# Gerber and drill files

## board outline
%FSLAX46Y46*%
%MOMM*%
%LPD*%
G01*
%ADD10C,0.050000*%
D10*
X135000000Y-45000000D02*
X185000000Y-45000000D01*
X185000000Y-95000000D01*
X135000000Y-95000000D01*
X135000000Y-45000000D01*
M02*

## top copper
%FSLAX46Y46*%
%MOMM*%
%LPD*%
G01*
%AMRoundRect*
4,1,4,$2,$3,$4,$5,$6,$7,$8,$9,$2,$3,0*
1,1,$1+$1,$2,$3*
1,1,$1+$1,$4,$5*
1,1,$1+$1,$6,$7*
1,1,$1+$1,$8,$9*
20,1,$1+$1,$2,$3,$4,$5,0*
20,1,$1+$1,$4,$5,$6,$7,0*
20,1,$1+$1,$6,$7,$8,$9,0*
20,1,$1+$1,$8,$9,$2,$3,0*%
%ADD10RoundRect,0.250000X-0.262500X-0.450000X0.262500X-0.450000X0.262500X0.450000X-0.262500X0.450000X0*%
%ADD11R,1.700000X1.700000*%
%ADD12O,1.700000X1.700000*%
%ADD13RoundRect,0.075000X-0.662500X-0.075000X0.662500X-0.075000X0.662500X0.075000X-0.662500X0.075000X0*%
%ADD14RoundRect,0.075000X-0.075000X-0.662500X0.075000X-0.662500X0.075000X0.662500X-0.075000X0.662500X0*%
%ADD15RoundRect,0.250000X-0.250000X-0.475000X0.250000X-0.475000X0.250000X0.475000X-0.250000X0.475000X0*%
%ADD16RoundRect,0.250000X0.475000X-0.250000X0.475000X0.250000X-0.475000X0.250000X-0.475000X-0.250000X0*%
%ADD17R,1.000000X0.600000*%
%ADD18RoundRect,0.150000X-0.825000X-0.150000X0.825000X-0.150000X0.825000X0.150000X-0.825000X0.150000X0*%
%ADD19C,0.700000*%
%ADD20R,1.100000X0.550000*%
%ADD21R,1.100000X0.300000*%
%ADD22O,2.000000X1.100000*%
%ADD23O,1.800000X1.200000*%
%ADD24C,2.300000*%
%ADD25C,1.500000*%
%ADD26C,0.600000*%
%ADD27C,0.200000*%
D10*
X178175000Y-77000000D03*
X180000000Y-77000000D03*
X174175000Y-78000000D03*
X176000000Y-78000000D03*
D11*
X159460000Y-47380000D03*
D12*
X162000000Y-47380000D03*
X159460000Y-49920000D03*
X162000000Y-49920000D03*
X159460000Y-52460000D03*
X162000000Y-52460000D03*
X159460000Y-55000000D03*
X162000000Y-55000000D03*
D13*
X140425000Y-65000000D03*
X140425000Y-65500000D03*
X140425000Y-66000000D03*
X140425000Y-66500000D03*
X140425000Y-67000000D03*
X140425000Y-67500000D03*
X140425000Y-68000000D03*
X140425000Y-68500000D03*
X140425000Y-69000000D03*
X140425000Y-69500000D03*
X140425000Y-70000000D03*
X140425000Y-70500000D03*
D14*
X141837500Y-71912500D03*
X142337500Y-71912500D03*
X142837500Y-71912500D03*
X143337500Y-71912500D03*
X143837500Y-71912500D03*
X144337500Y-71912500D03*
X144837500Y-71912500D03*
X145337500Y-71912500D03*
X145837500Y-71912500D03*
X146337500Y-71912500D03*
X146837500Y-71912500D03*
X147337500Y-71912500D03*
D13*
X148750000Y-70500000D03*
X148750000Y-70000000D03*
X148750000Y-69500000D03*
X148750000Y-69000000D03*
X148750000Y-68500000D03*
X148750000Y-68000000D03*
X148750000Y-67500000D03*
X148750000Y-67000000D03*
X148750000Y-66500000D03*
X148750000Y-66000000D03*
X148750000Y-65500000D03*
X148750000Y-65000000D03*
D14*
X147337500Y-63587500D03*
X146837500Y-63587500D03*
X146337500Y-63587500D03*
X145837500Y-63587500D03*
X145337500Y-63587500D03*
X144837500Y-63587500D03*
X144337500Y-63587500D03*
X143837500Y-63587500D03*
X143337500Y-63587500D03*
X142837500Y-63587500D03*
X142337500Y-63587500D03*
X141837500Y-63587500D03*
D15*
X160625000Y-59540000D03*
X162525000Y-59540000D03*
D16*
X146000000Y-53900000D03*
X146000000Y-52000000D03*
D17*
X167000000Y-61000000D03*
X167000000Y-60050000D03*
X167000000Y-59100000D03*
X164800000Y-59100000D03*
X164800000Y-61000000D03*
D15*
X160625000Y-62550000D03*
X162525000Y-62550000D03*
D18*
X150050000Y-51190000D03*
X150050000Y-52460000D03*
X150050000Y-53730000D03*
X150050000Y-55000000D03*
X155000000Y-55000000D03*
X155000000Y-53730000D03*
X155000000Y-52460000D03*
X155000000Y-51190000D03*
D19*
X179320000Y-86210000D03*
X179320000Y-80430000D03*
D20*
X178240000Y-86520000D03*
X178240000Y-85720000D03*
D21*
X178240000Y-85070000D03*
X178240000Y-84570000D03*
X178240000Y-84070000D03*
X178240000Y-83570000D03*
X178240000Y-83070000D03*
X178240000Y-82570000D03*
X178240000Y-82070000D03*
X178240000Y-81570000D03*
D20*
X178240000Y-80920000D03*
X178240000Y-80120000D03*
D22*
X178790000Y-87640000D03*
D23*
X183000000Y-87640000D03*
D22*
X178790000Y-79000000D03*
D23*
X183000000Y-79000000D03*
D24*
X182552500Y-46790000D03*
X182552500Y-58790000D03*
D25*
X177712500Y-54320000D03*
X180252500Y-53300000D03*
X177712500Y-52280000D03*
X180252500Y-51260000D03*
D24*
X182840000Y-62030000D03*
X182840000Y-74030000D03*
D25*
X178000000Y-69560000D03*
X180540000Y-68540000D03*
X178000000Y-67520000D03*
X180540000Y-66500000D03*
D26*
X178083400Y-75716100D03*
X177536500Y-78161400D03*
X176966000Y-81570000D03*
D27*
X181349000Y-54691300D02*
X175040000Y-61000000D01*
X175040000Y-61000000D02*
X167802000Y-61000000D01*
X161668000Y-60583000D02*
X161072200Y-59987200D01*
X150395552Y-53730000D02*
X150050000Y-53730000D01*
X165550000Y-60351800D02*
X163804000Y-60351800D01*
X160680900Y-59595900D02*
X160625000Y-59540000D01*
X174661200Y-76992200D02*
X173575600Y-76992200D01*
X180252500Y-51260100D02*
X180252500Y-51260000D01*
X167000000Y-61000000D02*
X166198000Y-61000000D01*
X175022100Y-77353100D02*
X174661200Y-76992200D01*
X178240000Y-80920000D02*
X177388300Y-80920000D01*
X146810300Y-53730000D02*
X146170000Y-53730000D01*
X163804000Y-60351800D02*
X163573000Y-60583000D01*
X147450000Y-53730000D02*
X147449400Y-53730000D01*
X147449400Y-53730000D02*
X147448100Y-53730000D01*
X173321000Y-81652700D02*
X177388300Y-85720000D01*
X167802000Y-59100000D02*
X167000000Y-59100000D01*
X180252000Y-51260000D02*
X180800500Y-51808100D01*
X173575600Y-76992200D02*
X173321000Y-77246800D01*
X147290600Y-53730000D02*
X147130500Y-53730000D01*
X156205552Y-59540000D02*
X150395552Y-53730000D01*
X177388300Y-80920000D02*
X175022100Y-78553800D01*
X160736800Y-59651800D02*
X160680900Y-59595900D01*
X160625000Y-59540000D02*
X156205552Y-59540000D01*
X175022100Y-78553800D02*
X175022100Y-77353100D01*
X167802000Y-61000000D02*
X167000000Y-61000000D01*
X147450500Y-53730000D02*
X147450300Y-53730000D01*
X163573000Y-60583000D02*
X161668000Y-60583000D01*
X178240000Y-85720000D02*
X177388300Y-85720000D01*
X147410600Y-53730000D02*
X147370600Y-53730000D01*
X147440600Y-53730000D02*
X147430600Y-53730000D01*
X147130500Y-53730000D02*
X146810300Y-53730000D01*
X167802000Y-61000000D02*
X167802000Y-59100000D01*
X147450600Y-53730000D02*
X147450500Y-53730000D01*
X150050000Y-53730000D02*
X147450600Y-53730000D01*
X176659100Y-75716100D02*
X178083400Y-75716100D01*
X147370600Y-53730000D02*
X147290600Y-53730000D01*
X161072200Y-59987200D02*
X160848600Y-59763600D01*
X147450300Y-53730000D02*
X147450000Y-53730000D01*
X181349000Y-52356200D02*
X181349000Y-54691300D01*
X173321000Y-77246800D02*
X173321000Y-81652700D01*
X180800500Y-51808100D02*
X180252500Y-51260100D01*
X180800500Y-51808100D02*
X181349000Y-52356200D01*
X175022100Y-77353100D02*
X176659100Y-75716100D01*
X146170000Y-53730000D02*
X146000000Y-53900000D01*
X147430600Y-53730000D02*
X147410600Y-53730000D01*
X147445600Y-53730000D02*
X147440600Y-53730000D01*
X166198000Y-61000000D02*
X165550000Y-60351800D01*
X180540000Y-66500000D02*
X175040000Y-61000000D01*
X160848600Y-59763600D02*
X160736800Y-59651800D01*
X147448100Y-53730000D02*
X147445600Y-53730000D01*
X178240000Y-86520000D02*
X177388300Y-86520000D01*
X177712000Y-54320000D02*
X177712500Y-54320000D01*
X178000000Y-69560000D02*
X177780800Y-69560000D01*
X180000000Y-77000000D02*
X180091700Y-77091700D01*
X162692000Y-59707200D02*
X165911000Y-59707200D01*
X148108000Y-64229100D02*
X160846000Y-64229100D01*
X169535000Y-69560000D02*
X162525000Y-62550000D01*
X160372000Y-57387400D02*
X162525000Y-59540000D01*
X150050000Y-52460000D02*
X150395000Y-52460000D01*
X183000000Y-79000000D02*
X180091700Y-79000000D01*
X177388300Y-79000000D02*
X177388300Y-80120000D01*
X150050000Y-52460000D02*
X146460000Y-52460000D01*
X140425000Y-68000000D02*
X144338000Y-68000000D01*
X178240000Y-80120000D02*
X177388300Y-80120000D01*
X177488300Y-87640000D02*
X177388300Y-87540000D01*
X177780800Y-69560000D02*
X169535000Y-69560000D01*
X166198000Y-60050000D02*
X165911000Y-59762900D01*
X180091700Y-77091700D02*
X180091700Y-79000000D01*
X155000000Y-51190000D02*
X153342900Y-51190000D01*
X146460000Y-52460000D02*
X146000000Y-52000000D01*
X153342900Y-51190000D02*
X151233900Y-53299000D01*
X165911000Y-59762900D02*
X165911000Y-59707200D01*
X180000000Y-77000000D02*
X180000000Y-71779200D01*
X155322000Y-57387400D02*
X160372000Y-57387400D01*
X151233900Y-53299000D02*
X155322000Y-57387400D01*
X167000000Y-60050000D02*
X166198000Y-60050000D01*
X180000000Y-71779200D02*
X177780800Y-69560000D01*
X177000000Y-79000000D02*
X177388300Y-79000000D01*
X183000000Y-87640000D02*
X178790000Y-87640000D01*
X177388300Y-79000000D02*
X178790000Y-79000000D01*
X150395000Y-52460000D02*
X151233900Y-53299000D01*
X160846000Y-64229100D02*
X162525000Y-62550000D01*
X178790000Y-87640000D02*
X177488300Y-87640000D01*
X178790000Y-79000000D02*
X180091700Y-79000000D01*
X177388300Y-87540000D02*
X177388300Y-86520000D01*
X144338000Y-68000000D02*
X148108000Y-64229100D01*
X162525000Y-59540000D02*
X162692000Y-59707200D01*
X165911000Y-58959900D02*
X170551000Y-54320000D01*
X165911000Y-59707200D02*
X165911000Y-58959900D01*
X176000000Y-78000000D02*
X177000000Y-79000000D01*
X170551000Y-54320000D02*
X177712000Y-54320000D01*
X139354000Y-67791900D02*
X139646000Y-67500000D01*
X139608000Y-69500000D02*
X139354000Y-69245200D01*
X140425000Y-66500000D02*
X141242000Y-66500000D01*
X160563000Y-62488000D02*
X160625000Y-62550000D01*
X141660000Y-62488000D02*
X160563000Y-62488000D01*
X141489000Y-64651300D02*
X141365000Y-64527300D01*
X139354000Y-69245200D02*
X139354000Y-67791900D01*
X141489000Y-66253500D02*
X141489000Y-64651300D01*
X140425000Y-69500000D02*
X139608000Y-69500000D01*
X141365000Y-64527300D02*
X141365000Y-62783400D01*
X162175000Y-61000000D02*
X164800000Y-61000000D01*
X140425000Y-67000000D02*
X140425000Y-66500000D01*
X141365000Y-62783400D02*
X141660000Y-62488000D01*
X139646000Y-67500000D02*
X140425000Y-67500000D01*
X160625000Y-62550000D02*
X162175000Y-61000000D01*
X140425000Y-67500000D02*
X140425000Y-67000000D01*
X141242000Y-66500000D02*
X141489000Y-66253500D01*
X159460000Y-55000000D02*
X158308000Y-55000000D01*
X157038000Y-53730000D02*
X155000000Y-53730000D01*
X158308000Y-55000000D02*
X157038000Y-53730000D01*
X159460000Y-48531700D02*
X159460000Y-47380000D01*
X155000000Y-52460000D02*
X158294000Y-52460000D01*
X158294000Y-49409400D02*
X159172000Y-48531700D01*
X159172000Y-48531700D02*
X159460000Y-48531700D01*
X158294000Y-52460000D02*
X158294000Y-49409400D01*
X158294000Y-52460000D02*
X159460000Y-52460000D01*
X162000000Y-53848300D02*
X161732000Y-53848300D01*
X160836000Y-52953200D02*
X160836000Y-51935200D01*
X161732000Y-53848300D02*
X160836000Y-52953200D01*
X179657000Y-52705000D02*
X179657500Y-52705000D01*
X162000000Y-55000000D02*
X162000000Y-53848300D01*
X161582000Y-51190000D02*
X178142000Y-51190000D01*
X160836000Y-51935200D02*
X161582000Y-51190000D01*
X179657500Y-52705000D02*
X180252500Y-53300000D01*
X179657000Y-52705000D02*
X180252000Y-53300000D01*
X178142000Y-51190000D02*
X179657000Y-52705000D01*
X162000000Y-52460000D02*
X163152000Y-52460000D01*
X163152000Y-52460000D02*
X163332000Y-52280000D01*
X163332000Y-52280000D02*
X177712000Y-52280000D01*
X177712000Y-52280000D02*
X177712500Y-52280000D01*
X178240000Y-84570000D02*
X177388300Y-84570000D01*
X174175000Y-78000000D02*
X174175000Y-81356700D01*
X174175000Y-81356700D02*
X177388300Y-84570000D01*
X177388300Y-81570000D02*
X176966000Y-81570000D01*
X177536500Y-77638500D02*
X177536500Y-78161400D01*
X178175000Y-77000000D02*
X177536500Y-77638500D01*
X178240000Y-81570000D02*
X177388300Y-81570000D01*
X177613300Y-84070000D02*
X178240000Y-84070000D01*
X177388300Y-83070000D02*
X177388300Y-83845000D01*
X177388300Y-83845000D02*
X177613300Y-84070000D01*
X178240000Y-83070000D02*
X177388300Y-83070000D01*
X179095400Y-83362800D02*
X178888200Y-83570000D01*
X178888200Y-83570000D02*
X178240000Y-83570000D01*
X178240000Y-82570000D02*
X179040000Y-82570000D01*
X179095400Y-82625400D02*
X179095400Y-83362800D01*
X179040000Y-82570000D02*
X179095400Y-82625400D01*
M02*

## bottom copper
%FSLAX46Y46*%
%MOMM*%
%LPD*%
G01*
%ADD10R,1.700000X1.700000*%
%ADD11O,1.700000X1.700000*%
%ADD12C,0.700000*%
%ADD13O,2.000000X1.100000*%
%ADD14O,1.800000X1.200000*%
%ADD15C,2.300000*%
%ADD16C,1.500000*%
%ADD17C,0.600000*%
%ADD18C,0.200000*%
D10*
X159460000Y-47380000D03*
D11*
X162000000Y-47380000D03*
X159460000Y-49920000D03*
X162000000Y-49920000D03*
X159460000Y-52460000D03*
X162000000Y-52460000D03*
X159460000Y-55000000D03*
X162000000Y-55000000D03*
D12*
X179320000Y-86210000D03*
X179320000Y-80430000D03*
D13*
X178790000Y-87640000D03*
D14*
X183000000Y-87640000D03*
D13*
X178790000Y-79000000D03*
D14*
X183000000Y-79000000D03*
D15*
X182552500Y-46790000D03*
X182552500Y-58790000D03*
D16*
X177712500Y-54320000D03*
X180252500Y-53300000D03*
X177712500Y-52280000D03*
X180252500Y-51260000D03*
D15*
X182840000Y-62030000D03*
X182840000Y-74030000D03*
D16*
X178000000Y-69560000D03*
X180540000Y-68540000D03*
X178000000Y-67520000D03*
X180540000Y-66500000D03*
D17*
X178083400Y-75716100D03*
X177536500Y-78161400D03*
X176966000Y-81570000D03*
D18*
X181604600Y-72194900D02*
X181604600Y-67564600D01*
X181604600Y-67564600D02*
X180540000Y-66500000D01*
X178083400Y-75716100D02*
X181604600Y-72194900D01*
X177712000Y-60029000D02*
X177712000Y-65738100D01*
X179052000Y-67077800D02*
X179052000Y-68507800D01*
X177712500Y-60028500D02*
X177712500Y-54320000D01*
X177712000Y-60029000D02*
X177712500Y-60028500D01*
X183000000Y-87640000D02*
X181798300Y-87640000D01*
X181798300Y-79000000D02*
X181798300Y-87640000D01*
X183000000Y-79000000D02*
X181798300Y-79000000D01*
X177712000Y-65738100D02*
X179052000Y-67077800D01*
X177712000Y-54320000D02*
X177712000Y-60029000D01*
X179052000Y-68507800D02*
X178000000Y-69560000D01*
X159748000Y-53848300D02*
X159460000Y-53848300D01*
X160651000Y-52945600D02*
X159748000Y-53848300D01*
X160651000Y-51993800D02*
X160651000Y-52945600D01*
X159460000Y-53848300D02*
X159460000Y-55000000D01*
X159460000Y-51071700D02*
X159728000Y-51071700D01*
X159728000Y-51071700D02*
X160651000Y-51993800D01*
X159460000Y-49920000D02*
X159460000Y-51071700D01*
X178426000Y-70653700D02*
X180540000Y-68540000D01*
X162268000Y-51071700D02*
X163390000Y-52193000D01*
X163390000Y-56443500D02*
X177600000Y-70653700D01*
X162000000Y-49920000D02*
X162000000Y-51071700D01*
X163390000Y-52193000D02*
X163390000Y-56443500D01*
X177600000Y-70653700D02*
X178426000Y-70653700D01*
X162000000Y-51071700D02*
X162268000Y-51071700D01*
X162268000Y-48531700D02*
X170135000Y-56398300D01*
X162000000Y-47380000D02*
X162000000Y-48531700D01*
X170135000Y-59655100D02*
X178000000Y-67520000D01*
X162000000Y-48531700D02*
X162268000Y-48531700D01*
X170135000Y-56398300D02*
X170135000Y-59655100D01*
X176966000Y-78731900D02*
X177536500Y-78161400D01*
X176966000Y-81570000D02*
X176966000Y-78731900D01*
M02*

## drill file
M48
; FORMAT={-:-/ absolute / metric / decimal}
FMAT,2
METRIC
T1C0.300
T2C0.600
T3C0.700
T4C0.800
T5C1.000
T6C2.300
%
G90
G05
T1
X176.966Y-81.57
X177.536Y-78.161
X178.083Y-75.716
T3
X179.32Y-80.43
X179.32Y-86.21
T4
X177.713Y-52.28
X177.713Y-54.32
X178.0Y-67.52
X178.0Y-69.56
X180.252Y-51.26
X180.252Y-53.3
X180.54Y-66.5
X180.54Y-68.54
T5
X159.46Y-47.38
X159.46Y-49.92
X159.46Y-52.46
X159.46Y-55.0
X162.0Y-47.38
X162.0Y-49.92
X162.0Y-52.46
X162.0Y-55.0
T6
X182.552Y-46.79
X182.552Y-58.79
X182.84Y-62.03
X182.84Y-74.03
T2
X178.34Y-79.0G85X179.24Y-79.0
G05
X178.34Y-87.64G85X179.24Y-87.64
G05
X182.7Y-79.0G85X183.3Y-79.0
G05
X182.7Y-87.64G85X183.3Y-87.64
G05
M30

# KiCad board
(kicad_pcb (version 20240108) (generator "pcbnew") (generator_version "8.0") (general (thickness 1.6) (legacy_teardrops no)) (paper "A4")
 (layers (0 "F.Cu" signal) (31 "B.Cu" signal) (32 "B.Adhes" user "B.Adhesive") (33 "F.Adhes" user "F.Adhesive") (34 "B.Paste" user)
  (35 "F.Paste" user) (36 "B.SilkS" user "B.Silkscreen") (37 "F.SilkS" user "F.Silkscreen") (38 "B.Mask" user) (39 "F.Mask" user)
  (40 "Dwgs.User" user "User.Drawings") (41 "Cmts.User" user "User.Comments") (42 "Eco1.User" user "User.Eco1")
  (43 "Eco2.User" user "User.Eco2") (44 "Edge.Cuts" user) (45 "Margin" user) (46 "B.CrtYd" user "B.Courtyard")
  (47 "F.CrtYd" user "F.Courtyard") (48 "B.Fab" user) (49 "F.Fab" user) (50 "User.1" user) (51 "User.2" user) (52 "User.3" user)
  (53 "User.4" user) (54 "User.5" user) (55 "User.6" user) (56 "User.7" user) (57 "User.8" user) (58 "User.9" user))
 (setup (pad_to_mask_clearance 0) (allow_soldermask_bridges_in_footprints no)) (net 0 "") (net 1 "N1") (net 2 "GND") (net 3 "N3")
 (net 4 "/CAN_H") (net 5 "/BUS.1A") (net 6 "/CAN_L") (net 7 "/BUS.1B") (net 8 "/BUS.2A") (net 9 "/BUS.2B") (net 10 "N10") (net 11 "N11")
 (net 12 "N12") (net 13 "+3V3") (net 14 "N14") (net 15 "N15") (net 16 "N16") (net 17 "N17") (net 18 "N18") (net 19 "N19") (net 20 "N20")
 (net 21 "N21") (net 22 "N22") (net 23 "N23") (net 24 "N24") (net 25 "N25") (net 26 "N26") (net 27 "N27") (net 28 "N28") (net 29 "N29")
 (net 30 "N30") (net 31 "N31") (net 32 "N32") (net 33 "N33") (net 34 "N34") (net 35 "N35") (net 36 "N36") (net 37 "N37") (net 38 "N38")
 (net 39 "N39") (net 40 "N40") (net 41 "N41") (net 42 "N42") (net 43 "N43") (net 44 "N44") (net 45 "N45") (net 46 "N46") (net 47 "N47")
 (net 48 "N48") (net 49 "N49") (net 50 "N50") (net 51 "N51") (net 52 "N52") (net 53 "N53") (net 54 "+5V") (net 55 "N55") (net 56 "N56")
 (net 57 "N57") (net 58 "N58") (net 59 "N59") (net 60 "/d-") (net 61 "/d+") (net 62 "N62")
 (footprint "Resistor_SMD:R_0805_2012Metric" (layer "F.Cu") (at 179.0875 77)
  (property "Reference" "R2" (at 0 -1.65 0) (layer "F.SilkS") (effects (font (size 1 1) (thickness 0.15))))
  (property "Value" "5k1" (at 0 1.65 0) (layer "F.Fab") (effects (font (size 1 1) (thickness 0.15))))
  (pad "1" smd roundrect (at -0.9125 0) (size 1.025 1.4) (layers "F.Cu" "F.Paste" "F.Mask") (roundrect_rratio 0.243902) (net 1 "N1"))
  (pad "2" smd roundrect (at 0.9125 0) (size 1.025 1.4) (layers "F.Cu" "F.Paste" "F.Mask") (roundrect_rratio 0.243902) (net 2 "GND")))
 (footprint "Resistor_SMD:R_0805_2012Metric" (layer "F.Cu") (at 175.0875 78)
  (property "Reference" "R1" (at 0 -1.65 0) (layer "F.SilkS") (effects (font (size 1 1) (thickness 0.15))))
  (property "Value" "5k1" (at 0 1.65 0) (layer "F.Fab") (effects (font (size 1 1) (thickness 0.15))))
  (pad "1" smd roundrect (at -0.9125 0) (size 1.025 1.4) (layers "F.Cu" "F.Paste" "F.Mask") (roundrect_rratio 0.243902) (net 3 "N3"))
  (pad "2" smd roundrect (at 0.9125 0) (size 1.025 1.4) (layers "F.Cu" "F.Paste" "F.Mask") (roundrect_rratio 0.243902) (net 2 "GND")))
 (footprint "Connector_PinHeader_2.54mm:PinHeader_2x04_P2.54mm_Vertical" (layer "F.Cu") (at 159.46 47.38)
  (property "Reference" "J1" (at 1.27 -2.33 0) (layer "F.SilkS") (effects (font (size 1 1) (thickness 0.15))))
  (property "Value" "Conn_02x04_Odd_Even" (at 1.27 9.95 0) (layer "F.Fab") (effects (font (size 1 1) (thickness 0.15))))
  (pad "1" thru_hole rect (at 0 0) (size 1.7 1.7) (drill 1) (layers "*.Cu" "*.Mask") (remove_unused_layers no) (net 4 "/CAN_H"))
  (pad "2" thru_hole oval (at 2.54 0) (size 1.7 1.7) (drill 1) (layers "*.Cu" "*.Mask") (remove_unused_layers no) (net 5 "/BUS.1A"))
  (pad "3" thru_hole oval (at 0 2.54) (size 1.7 1.7) (drill 1) (layers "*.Cu" "*.Mask") (remove_unused_layers no) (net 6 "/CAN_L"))
  (pad "4" thru_hole oval (at 2.54 2.54) (size 1.7 1.7) (drill 1) (layers "*.Cu" "*.Mask") (remove_unused_layers no) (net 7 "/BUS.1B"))
  (pad "5" thru_hole oval (at 0 5.08) (size 1.7 1.7) (drill 1) (layers "*.Cu" "*.Mask") (remove_unused_layers no) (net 4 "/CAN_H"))
  (pad "6" thru_hole oval (at 2.54 5.08) (size 1.7 1.7) (drill 1) (layers "*.Cu" "*.Mask") (remove_unused_layers no) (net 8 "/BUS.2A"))
  (pad "7" thru_hole oval (at 0 7.62) (size 1.7 1.7) (drill 1) (layers "*.Cu" "*.Mask") (remove_unused_layers no) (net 6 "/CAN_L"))
  (pad "8" thru_hole oval (at 2.54 7.62) (size 1.7 1.7) (drill 1) (layers "*.Cu" "*.Mask") (remove_unused_layers no) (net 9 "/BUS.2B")))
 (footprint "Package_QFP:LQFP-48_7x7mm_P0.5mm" (layer "F.Cu") (at 144.5875 67.75)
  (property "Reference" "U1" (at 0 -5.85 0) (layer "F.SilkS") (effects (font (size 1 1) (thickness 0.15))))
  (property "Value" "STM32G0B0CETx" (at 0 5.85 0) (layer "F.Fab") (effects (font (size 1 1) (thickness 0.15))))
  (pad "1" smd roundrect (at -4.1625 -2.75) (size 1.475 0.3) (layers "F.Cu" "F.Paste" "F.Mask") (roundrect_rratio 0.25) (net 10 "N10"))
  (pad "2" smd roundrect (at -4.1625 -2.25) (size 1.475 0.3) (layers "F.Cu" "F.Paste" "F.Mask") (roundrect_rratio 0.25) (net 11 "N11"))
  (pad "3" smd roundrect (at -4.1625 -1.75) (size 1.475 0.3) (layers "F.Cu" "F.Paste" "F.Mask") (roundrect_rratio 0.25) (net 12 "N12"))
  (pad "4" smd roundrect (at -4.1625 -1.25) (size 1.475 0.3) (layers "F.Cu" "F.Paste" "F.Mask") (roundrect_rratio 0.25) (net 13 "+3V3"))
  (pad "5" smd roundrect (at -4.1625 -0.75) (size 1.475 0.3) (layers "F.Cu" "F.Paste" "F.Mask") (roundrect_rratio 0.25) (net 13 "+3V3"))
  (pad "6" smd roundrect (at -4.1625 -0.25) (size 1.475 0.3) (layers "F.Cu" "F.Paste" "F.Mask") (roundrect_rratio 0.25) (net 13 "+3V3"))
  (pad "7" smd roundrect (at -4.1625 0.25) (size 1.475 0.3) (layers "F.Cu" "F.Paste" "F.Mask") (roundrect_rratio 0.25) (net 2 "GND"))
  (pad "8" smd roundrect (at -4.1625 0.75) (size 1.475 0.3) (layers "F.Cu" "F.Paste" "F.Mask") (roundrect_rratio 0.25) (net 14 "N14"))
  (pad "9" smd roundrect (at -4.1625 1.25) (size 1.475 0.3) (layers "F.Cu" "F.Paste" "F.Mask") (roundrect_rratio 0.25) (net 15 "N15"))
  (pad "10" smd roundrect (at -4.1625 1.75) (size 1.475 0.3) (layers "F.Cu" "F.Paste" "F.Mask") (roundrect_rratio 0.25) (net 13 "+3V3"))
  (pad "11" smd roundrect (at -4.1625 2.25) (size 1.475 0.3) (layers "F.Cu" "F.Paste" "F.Mask") (roundrect_rratio 0.25) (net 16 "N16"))
  (pad "12" smd roundrect (at -4.1625 2.75) (size 1.475 0.3) (layers "F.Cu" "F.Paste" "F.Mask") (roundrect_rratio 0.25) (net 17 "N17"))
  (pad "13" smd roundrect (at -2.75 4.1625) (size 0.3 1.475) (layers "F.Cu" "F.Paste" "F.Mask") (roundrect_rratio 0.25) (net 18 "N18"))
  (pad "14" smd roundrect (at -2.25 4.1625) (size 0.3 1.475) (layers "F.Cu" "F.Paste" "F.Mask") (roundrect_rratio 0.25) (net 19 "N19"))
  (pad "15" smd roundrect (at -1.75 4.1625) (size 0.3 1.475) (layers "F.Cu" "F.Paste" "F.Mask") (roundrect_rratio 0.25) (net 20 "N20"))
  (pad "16" smd roundrect (at -1.25 4.1625) (size 0.3 1.475) (layers "F.Cu" "F.Paste" "F.Mask") (roundrect_rratio 0.25) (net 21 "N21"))
  (pad "17" smd roundrect (at -0.75 4.1625) (size 0.3 1.475) (layers "F.Cu" "F.Paste" "F.Mask") (roundrect_rratio 0.25) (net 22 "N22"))
  (pad "18" smd roundrect (at -0.25 4.1625) (size 0.3 1.475) (layers "F.Cu" "F.Paste" "F.Mask") (roundrect_rratio 0.25) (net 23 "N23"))
  (pad "19" smd roundrect (at 0.25 4.1625) (size 0.3 1.475) (layers "F.Cu" "F.Paste" "F.Mask") (roundrect_rratio 0.25) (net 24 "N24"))
  (pad "20" smd roundrect (at 0.75 4.1625) (size 0.3 1.475) (layers "F.Cu" "F.Paste" "F.Mask") (roundrect_rratio 0.25) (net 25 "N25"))
  (pad "21" smd roundrect (at 1.25 4.1625) (size 0.3 1.475) (layers "F.Cu" "F.Paste" "F.Mask") (roundrect_rratio 0.25) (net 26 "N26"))
  (pad "22" smd roundrect (at 1.75 4.1625) (size 0.3 1.475) (layers "F.Cu" "F.Paste" "F.Mask") (roundrect_rratio 0.25) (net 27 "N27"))
  (pad "23" smd roundrect (at 2.25 4.1625) (size 0.3 1.475) (layers "F.Cu" "F.Paste" "F.Mask") (roundrect_rratio 0.25) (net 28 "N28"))
  (pad "24" smd roundrect (at 2.75 4.1625) (size 0.3 1.475) (layers "F.Cu" "F.Paste" "F.Mask") (roundrect_rratio 0.25) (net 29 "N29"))
  (pad "25" smd roundrect (at 4.1625 2.75) (size 1.475 0.3) (layers "F.Cu" "F.Paste" "F.Mask") (roundrect_rratio 0.25) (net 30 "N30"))
  (pad "26" smd roundrect (at 4.1625 2.25) (size 1.475 0.3) (layers "F.Cu" "F.Paste" "F.Mask") (roundrect_rratio 0.25) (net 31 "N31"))
  (pad "27" smd roundrect (at 4.1625 1.75) (size 1.475 0.3) (layers "F.Cu" "F.Paste" "F.Mask") (roundrect_rratio 0.25) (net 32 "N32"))
  (pad "28" smd roundrect (at 4.1625 1.25) (size 1.475 0.3) (layers "F.Cu" "F.Paste" "F.Mask") (roundrect_rratio 0.25) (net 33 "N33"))
  (pad "29" smd roundrect (at 4.1625 0.75) (size 1.475 0.3) (layers "F.Cu" "F.Paste" "F.Mask") (roundrect_rratio 0.25) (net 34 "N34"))
  (pad "30" smd roundrect (at 4.1625 0.25) (size 1.475 0.3) (layers "F.Cu" "F.Paste" "F.Mask") (roundrect_rratio 0.25) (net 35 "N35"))
  (pad "31" smd roundrect (at 4.1625 -0.25) (size 1.475 0.3) (layers "F.Cu" "F.Paste" "F.Mask") (roundrect_rratio 0.25) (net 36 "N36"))
  (pad "32" smd roundrect (at 4.1625 -0.75) (size 1.475 0.3) (layers "F.Cu" "F.Paste" "F.Mask") (roundrect_rratio 0.25) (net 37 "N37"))
  (pad "33" smd roundrect (at 4.1625 -1.25) (size 1.475 0.3) (layers "F.Cu" "F.Paste" "F.Mask") (roundrect_rratio 0.25) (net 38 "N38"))
  (pad "34" smd roundrect (at 4.1625 -1.75) (size 1.475 0.3) (layers "F.Cu" "F.Paste" "F.Mask") (roundrect_rratio 0.25) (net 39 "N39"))
  (pad "35" smd roundrect (at 4.1625 -2.25) (size 1.475 0.3) (layers "F.Cu" "F.Paste" "F.Mask") (roundrect_rratio 0.25) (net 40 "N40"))
  (pad "36" smd roundrect (at 4.1625 -2.75) (size 1.475 0.3) (layers "F.Cu" "F.Paste" "F.Mask") (roundrect_rratio 0.25) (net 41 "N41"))
  (pad "37" smd roundrect (at 2.75 -4.1625) (size 0.3 1.475) (layers "F.Cu" "F.Paste" "F.Mask") (roundrect_rratio 0.25) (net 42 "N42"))
  (pad "38" smd roundrect (at 2.25 -4.1625) (size 0.3 1.475) (layers "F.Cu" "F.Paste" "F.Mask") (roundrect_rratio 0.25) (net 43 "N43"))
  (pad "39" smd roundrect (at 1.75 -4.1625) (size 0.3 1.475) (layers "F.Cu" "F.Paste" "F.Mask") (roundrect_rratio 0.25) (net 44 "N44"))
  (pad "40" smd roundrect (at 1.25 -4.1625) (size 0.3 1.475) (layers "F.Cu" "F.Paste" "F.Mask") (roundrect_rratio 0.25) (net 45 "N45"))
  (pad "41" smd roundrect (at 0.75 -4.1625) (size 0.3 1.475) (layers "F.Cu" "F.Paste" "F.Mask") (roundrect_rratio 0.25) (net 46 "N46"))
  (pad "42" smd roundrect (at 0.25 -4.1625) (size 0.3 1.475) (layers "F.Cu" "F.Paste" "F.Mask") (roundrect_rratio 0.25) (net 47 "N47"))
  (pad "43" smd roundrect (at -0.25 -4.1625) (size 0.3 1.475) (layers "F.Cu" "F.Paste" "F.Mask") (roundrect_rratio 0.25) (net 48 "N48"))
  (pad "44" smd roundrect (at -0.75 -4.1625) (size 0.3 1.475) (layers "F.Cu" "F.Paste" "F.Mask") (roundrect_rratio 0.25) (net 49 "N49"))
  (pad "45" smd roundrect (at -1.25 -4.1625) (size 0.3 1.475) (layers "F.Cu" "F.Paste" "F.Mask") (roundrect_rratio 0.25) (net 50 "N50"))
  (pad "46" smd roundrect (at -1.75 -4.1625) (size 0.3 1.475) (layers "F.Cu" "F.Paste" "F.Mask") (roundrect_rratio 0.25) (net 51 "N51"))
  (pad "47" smd roundrect (at -2.25 -4.1625) (size 0.3 1.475) (layers "F.Cu" "F.Paste" "F.Mask") (roundrect_rratio 0.25) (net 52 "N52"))
  (pad "48" smd roundrect (at -2.75 -4.1625) (size 0.3 1.475) (layers "F.Cu" "F.Paste" "F.Mask") (roundrect_rratio 0.25) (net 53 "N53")))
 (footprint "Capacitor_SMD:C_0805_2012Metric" (layer "F.Cu") (at 161.575 59.54)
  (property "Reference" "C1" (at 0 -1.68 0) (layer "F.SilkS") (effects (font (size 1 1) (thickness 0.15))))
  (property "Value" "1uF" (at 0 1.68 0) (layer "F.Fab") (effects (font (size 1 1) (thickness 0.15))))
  (pad "1" smd roundrect (at -0.95 0) (size 1 1.45) (layers "F.Cu" "F.Paste" "F.Mask") (roundrect_rratio 0.25) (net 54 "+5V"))
  (pad "2" smd roundrect (at 0.95 0) (size 1 1.45) (layers "F.Cu" "F.Paste" "F.Mask") (roundrect_rratio 0.25) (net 2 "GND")))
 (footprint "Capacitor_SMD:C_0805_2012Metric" (layer "F.Cu") (at 146 52.95 90)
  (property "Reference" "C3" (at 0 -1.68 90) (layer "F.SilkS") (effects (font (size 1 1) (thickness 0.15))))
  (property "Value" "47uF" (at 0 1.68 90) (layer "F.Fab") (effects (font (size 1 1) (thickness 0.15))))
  (pad "1" smd roundrect (at -0.95 0 90) (size 1 1.45) (layers "F.Cu" "F.Paste" "F.Mask") (roundrect_rratio 0.25) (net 54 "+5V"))
  (pad "2" smd roundrect (at 0.95 0 90) (size 1 1.45) (layers "F.Cu" "F.Paste" "F.Mask") (roundrect_rratio 0.25) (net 2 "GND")))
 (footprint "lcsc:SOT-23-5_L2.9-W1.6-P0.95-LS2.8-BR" (layer "F.Cu") (at 165.9 60.05)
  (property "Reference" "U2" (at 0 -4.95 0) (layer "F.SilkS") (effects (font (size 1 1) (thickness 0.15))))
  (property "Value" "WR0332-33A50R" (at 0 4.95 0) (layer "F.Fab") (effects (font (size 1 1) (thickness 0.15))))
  (pad "1" smd rect (at 1.1 0.95 90) (size 0.6 1) (layers "F.Cu" "F.Paste" "F.Mask") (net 54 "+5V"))
  (pad "2" smd rect (at 1.1 0 90) (size 0.6 1) (layers "F.Cu" "F.Paste" "F.Mask") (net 2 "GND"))
  (pad "3" smd rect (at 1.1 -0.95 90) (size 0.6 1) (layers "F.Cu" "F.Paste" "F.Mask") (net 54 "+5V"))
  (pad "4" smd rect (at -1.1 -0.95 90) (size 0.6 1) (layers "F.Cu" "F.Paste" "F.Mask") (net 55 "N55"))
  (pad "5" smd rect (at -1.1 0.95 90) (size 0.6 1) (layers "F.Cu" "F.Paste" "F.Mask") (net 13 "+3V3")))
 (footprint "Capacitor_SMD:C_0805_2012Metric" (layer "F.Cu") (at 161.575 62.55)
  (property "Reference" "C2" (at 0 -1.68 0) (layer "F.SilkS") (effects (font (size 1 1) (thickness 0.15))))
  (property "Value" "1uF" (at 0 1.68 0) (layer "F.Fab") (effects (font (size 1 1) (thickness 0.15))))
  (pad "1" smd roundrect (at -0.95 0) (size 1 1.45) (layers "F.Cu" "F.Paste" "F.Mask") (roundrect_rratio 0.25) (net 13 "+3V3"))
  (pad "2" smd roundrect (at 0.95 0) (size 1 1.45) (layers "F.Cu" "F.Paste" "F.Mask") (roundrect_rratio 0.25) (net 2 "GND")))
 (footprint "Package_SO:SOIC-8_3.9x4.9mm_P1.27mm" (layer "F.Cu") (at 152.525 53.095)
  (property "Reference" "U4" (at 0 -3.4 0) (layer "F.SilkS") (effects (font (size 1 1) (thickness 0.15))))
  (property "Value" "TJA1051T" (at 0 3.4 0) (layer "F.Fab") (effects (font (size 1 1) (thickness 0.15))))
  (pad "1" smd roundrect (at -2.475 -1.905) (size 1.95 0.6) (layers "F.Cu" "F.Paste" "F.Mask") (roundrect_rratio 0.25) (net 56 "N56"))
  (pad "2" smd roundrect (at -2.475 -0.635) (size 1.95 0.6) (layers "F.Cu" "F.Paste" "F.Mask") (roundrect_rratio 0.25) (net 2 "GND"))
  (pad "3" smd roundrect (at -2.475 0.635) (size 1.95 0.6) (layers "F.Cu" "F.Paste" "F.Mask") (roundrect_rratio 0.25) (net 54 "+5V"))
  (pad "4" smd roundrect (at -2.475 1.905) (size 1.95 0.6) (layers "F.Cu" "F.Paste" "F.Mask") (roundrect_rratio 0.25) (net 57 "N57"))
  (pad "5" smd roundrect (at 2.475 1.905) (size 1.95 0.6) (layers "F.Cu" "F.Paste" "F.Mask") (roundrect_rratio 0.25) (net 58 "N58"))
  (pad "6" smd roundrect (at 2.475 0.635) (size 1.95 0.6) (layers "F.Cu" "F.Paste" "F.Mask") (roundrect_rratio 0.25) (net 6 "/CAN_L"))
  (pad "7" smd roundrect (at 2.475 -0.635) (size 1.95 0.6) (layers "F.Cu" "F.Paste" "F.Mask") (roundrect_rratio 0.25) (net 4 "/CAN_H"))
  (pad "8" smd roundrect (at 2.475 -1.905) (size 1.95 0.6) (layers "F.Cu" "F.Paste" "F.Mask") (roundrect_rratio 0.25) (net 2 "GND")))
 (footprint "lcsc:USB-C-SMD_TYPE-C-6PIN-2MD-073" (layer "F.Cu") (at 180.62 83.32 90)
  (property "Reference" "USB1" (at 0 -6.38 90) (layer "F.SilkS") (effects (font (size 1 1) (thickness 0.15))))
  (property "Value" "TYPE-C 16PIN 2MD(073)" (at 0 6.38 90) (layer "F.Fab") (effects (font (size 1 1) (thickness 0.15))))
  (pad "" thru_hole circle (at -2.89 -1.3 90) (size 0.7 0.7) (drill 0.7) (layers "*.Cu" "*.Mask") (remove_unused_layers no))
  (pad "" thru_hole circle (at 2.89 -1.3 90) (size 0.7 0.7) (drill 0.7) (layers "*.Cu" "*.Mask") (remove_unused_layers no))
  (pad "1" smd rect (at -3.2 -2.38 90) (size 0.55 1.1) (layers "F.Cu" "F.Paste" "F.Mask") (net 2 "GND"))
  (pad "2" smd rect (at -2.4 -2.38 90) (size 0.55 1.1) (layers "F.Cu" "F.Paste" "F.Mask") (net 54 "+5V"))
  (pad "3" smd rect (at -1.75 -2.38 90) (size 0.3 1.1) (layers "F.Cu" "F.Paste" "F.Mask") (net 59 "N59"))
  (pad "4" smd rect (at -1.25 -2.38 90) (size 0.3 1.1) (layers "F.Cu" "F.Paste" "F.Mask") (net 3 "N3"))
  (pad "5" smd rect (at -0.75 -2.38 90) (size 0.3 1.1) (layers "F.Cu" "F.Paste" "F.Mask") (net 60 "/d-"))
  (pad "6" smd rect (at -0.25 -2.38 90) (size 0.3 1.1) (layers "F.Cu" "F.Paste" "F.Mask") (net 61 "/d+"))
  (pad "7" smd rect (at 0.25 -2.38 90) (size 0.3 1.1) (layers "F.Cu" "F.Paste" "F.Mask") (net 60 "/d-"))
  (pad "8" smd rect (at 0.75 -2.38 90) (size 0.3 1.1) (layers "F.Cu" "F.Paste" "F.Mask") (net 61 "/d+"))
  (pad "9" smd rect (at 1.25 -2.38 90) (size 0.3 1.1) (layers "F.Cu" "F.Paste" "F.Mask") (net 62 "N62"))
  (pad "10" smd rect (at 1.75 -2.38 90) (size 0.3 1.1) (layers "F.Cu" "F.Paste" "F.Mask") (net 1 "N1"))
  (pad "11" smd rect (at 2.4 -2.38 90) (size 0.55 1.1) (layers "F.Cu" "F.Paste" "F.Mask") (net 54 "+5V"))
  (pad "12" smd rect (at 3.2 -2.38 90) (size 0.55 1.1) (layers "F.Cu" "F.Paste" "F.Mask") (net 2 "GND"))
  (pad "13" thru_hole oval (at -4.32 -1.83 90) (size 1.1 2) (drill oval 0.599999 1.499997) (layers "*.Cu" "*.Mask")
   (remove_unused_layers no) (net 2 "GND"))
  (pad "13" thru_hole oval (at -4.32 2.38 90) (size 1.2 1.8) (drill oval 0.599999 1.199998) (layers "*.Cu" "*.Mask")
   (remove_unused_layers no) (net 2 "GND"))
  (pad "14" thru_hole oval (at 4.32 -1.83 90) (size 1.1 2) (drill oval 0.599999 1.500022) (layers "*.Cu" "*.Mask") (remove_unused_layers no)
   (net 2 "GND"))
  (pad "14" thru_hole oval (at 4.32 2.38 90) (size 1.2 1.8) (drill oval 0.599999 1.199998) (layers "*.Cu" "*.Mask")
   (remove_unused_layers no) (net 2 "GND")))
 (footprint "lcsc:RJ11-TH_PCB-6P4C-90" (layer "F.Cu") (at 178.9825 52.79 -90)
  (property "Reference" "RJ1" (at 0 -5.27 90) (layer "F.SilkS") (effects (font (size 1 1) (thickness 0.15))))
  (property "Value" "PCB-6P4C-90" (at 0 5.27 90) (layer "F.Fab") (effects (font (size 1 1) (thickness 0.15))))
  (pad "" thru_hole circle (at -6 -3.57 270) (size 2.3 2.3) (drill 2.3) (layers "*.Cu" "*.Mask") (remove_unused_layers no))
  (pad "" thru_hole circle (at 6 -3.57 270) (size 2.3 2.3) (drill 2.3) (layers "*.Cu" "*.Mask") (remove_unused_layers no))
  (pad "1" thru_hole circle (at 1.53 1.27 270) (size 1.5 1.5) (drill 0.799998) (layers "*.Cu" "*.Mask") (remove_unused_layers no)
   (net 2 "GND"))
  (pad "2" thru_hole circle (at 0.51 -1.27 270) (size 1.5 1.5) (drill 0.799998) (layers "*.Cu" "*.Mask") (remove_unused_layers no)
   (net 9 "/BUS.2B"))
  (pad "3" thru_hole circle (at -0.51 1.27 270) (size 1.5 1.5) (drill 0.799998) (layers "*.Cu" "*.Mask") (remove_unused_layers no)
   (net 8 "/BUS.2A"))
  (pad "4" thru_hole circle (at -1.53 -1.27 270) (size 1.5 1.5) (drill 0.799998) (layers "*.Cu" "*.Mask") (remove_unused_layers no)
   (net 54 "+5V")))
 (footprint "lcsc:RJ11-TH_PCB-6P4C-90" (layer "F.Cu") (at 179.27 68.03 -90)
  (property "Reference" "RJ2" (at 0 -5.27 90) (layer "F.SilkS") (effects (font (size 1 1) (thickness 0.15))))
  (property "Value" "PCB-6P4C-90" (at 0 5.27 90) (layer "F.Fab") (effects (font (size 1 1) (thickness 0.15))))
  (pad "" thru_hole circle (at -6 -3.57 270) (size 2.3 2.3) (drill 2.3) (layers "*.Cu" "*.Mask") (remove_unused_layers no))
  (pad "" thru_hole circle (at 6 -3.57 270) (size 2.3 2.3) (drill 2.3) (layers "*.Cu" "*.Mask") (remove_unused_layers no))
  (pad "1" thru_hole circle (at 1.53 1.27 270) (size 1.5 1.5) (drill 0.799998) (layers "*.Cu" "*.Mask") (remove_unused_layers no)
   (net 2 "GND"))
  (pad "2" thru_hole circle (at 0.51 -1.27 270) (size 1.5 1.5) (drill 0.799998) (layers "*.Cu" "*.Mask") (remove_unused_layers no)
   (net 7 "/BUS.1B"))
  (pad "3" thru_hole circle (at -0.51 1.27 270) (size 1.5 1.5) (drill 0.799998) (layers "*.Cu" "*.Mask") (remove_unused_layers no)
   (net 5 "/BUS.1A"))
  (pad "4" thru_hole circle (at -1.53 -1.27 270) (size 1.5 1.5) (drill 0.799998) (layers "*.Cu" "*.Mask") (remove_unused_layers no)
   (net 54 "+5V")))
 (gr_rect (start 135 45) (end 185 95) (stroke (width 0.05) (type default)) (fill none) (layer "Edge.Cuts"))
 (segment (start 181.349 54.6913) (end 175.04 61) (width 0.2) (layer "F.Cu") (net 54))
 (segment (start 175.04 61) (end 167.802 61) (width 0.2) (layer "F.Cu") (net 54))
 (segment (start 161.668 60.583) (end 161.0722 59.9872) (width 0.2) (layer "F.Cu") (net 54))
 (segment (start 150.395552 53.73) (end 150.05 53.73) (width 0.2) (layer "F.Cu") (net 54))
 (segment (start 165.55 60.3518) (end 163.804 60.3518) (width 0.2) (layer "F.Cu") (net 54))
 (segment (start 160.6809 59.5959) (end 160.625 59.54) (width 0.2) (layer "F.Cu") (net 54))
 (segment (start 174.6612 76.9922) (end 173.5756 76.9922) (width 0.2) (layer "F.Cu") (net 54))
 (segment (start 180.2525 51.2601) (end 180.2525 51.26) (width 0.2) (layer "F.Cu") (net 54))
 (segment (start 167 61) (end 166.198 61) (width 0.2) (layer "F.Cu") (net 54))
 (segment (start 175.0221 77.3531) (end 174.6612 76.9922) (width 0.2) (layer "F.Cu") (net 54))
 (segment (start 178.24 80.92) (end 177.3883 80.92) (width 0.2) (layer "F.Cu") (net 54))
 (segment (start 146.8103 53.73) (end 146.17 53.73) (width 0.2) (layer "F.Cu") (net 54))
 (segment (start 163.804 60.3518) (end 163.573 60.583) (width 0.2) (layer "F.Cu") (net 54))
 (segment (start 147.45 53.73) (end 147.4494 53.73) (width 0.2) (layer "F.Cu") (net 54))
 (segment (start 147.4494 53.73) (end 147.4481 53.73) (width 0.2) (layer "F.Cu") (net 54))
 (segment (start 173.321 81.6527) (end 177.3883 85.72) (width 0.2) (layer "F.Cu") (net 54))
 (segment (start 167.802 59.1) (end 167 59.1) (width 0.2) (layer "F.Cu") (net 54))
 (segment (start 180.252 51.26) (end 180.8005 51.8081) (width 0.2) (layer "F.Cu") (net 54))
 (segment (start 173.5756 76.9922) (end 173.321 77.2468) (width 0.2) (layer "F.Cu") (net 54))
 (segment (start 147.2906 53.73) (end 147.1305 53.73) (width 0.2) (layer "F.Cu") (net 54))
 (segment (start 156.205552 59.54) (end 150.395552 53.73) (width 0.2) (layer "F.Cu") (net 54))
 (segment (start 177.3883 80.92) (end 175.0221 78.5538) (width 0.2) (layer "F.Cu") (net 54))
 (segment (start 160.7368 59.6518) (end 160.6809 59.5959) (width 0.2) (layer "F.Cu") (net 54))
 (segment (start 160.625 59.54) (end 156.205552 59.54) (width 0.2) (layer "F.Cu") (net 54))
 (segment (start 175.0221 78.5538) (end 175.0221 77.3531) (width 0.2) (layer "F.Cu") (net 54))
 (segment (start 167.802 61) (end 167 61) (width 0.2) (layer "F.Cu") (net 54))
 (segment (start 147.4505 53.73) (end 147.4503 53.73) (width 0.2) (layer "F.Cu") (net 54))
 (segment (start 163.573 60.583) (end 161.668 60.583) (width 0.2) (layer "F.Cu") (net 54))
 (segment (start 178.24 85.72) (end 177.3883 85.72) (width 0.2) (layer "F.Cu") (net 54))
 (segment (start 147.4106 53.73) (end 147.3706 53.73) (width 0.2) (layer "F.Cu") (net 54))
 (segment (start 147.4406 53.73) (end 147.4306 53.73) (width 0.2) (layer "F.Cu") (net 54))
 (segment (start 147.1305 53.73) (end 146.8103 53.73) (width 0.2) (layer "F.Cu") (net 54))
 (segment (start 167.802 61) (end 167.802 59.1) (width 0.2) (layer "F.Cu") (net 54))
 (segment (start 147.4506 53.73) (end 147.4505 53.73) (width 0.2) (layer "F.Cu") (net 54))
 (segment (start 150.05 53.73) (end 147.4506 53.73) (width 0.2) (layer "F.Cu") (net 54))
 (segment (start 176.6591 75.7161) (end 178.0834 75.7161) (width 0.2) (layer "F.Cu") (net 54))
 (segment (start 147.3706 53.73) (end 147.2906 53.73) (width 0.2) (layer "F.Cu") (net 54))
 (segment (start 161.0722 59.9872) (end 160.8486 59.7636) (width 0.2) (layer "F.Cu") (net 54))
 (segment (start 147.4503 53.73) (end 147.45 53.73) (width 0.2) (layer "F.Cu") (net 54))
 (segment (start 181.349 52.3562) (end 181.349 54.6913) (width 0.2) (layer "F.Cu") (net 54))
 (segment (start 173.321 77.2468) (end 173.321 81.6527) (width 0.2) (layer "F.Cu") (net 54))
 (segment (start 180.8005 51.8081) (end 180.2525 51.2601) (width 0.2) (layer "F.Cu") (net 54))
 (segment (start 180.8005 51.8081) (end 181.349 52.3562) (width 0.2) (layer "F.Cu") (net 54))
 (segment (start 175.0221 77.3531) (end 176.6591 75.7161) (width 0.2) (layer "F.Cu") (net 54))
 (segment (start 146.17 53.73) (end 146 53.9) (width 0.2) (layer "F.Cu") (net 54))
 (segment (start 147.4306 53.73) (end 147.4106 53.73) (width 0.2) (layer "F.Cu") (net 54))
 (segment (start 147.4456 53.73) (end 147.4406 53.73) (width 0.2) (layer "F.Cu") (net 54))
 (segment (start 166.198 61) (end 165.55 60.3518) (width 0.2) (layer "F.Cu") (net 54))
 (segment (start 180.54 66.5) (end 175.04 61) (width 0.2) (layer "F.Cu") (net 54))
 (segment (start 160.8486 59.7636) (end 160.7368 59.6518) (width 0.2) (layer "F.Cu") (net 54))
 (segment (start 147.4481 53.73) (end 147.4456 53.73) (width 0.2) (layer "F.Cu") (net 54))
 (via (at 178.0834 75.7161) (size 0.6) (drill 0.3) (layers "F.Cu" "B.Cu") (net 54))
 (segment (start 181.6046 72.1949) (end 181.6046 67.5646) (width 0.2) (layer "B.Cu") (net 54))
 (segment (start 181.6046 67.5646) (end 180.54 66.5) (width 0.2) (layer "B.Cu") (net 54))
 (segment (start 178.0834 75.7161) (end 181.6046 72.1949) (width 0.2) (layer "B.Cu") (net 54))
 (segment (start 178.24 86.52) (end 177.3883 86.52) (width 0.2) (layer "F.Cu") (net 2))
 (segment (start 177.712 54.32) (end 177.7125 54.32) (width 0.2) (layer "F.Cu") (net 2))
 (segment (start 178 69.56) (end 177.7808 69.56) (width 0.2) (layer "F.Cu") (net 2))
 (segment (start 180 77) (end 180.0917 77.0917) (width 0.2) (layer "F.Cu") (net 2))
 (segment (start 162.692 59.7072) (end 165.911 59.7072) (width 0.2) (layer "F.Cu") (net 2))
 (segment (start 148.108 64.2291) (end 160.846 64.2291) (width 0.2) (layer "F.Cu") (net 2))
 (segment (start 169.535 69.56) (end 162.525 62.55) (width 0.2) (layer "F.Cu") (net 2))
 (segment (start 160.372 57.3874) (end 162.525 59.54) (width 0.2) (layer "F.Cu") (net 2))
 (segment (start 150.05 52.46) (end 150.395 52.46) (width 0.2) (layer "F.Cu") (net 2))
 (segment (start 183 79) (end 180.0917 79) (width 0.2) (layer "F.Cu") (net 2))
 (segment (start 177.3883 79) (end 177.3883 80.12) (width 0.2) (layer "F.Cu") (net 2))
 (segment (start 150.05 52.46) (end 146.46 52.46) (width 0.2) (layer "F.Cu") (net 2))
 (segment (start 140.425 68) (end 144.338 68) (width 0.2) (layer "F.Cu") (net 2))
 (segment (start 178.24 80.12) (end 177.3883 80.12) (width 0.2) (layer "F.Cu") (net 2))
 (segment (start 177.4883 87.64) (end 177.3883 87.54) (width 0.2) (layer "F.Cu") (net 2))
 (segment (start 177.7808 69.56) (end 169.535 69.56) (width 0.2) (layer "F.Cu") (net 2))
 (segment (start 166.198 60.05) (end 165.911 59.7629) (width 0.2) (layer "F.Cu") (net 2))
 (segment (start 180.0917 77.0917) (end 180.0917 79) (width 0.2) (layer "F.Cu") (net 2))
 (segment (start 155 51.19) (end 153.3429 51.19) (width 0.2) (layer "F.Cu") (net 2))
 (segment (start 146.46 52.46) (end 146 52) (width 0.2) (layer "F.Cu") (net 2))
 (segment (start 153.3429 51.19) (end 151.2339 53.299) (width 0.2) (layer "F.Cu") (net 2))
 (segment (start 165.911 59.7629) (end 165.911 59.7072) (width 0.2) (layer "F.Cu") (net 2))
 (segment (start 180 77) (end 180 71.7792) (width 0.2) (layer "F.Cu") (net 2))
 (segment (start 155.322 57.3874) (end 160.372 57.3874) (width 0.2) (layer "F.Cu") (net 2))
 (segment (start 151.2339 53.299) (end 155.322 57.3874) (width 0.2) (layer "F.Cu") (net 2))
 (segment (start 167 60.05) (end 166.198 60.05) (width 0.2) (layer "F.Cu") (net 2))
 (segment (start 180 71.7792) (end 177.7808 69.56) (width 0.2) (layer "F.Cu") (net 2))
 (segment (start 177 79) (end 177.3883 79) (width 0.2) (layer "F.Cu") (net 2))
 (segment (start 183 87.64) (end 178.79 87.64) (width 0.2) (layer "F.Cu") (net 2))
 (segment (start 177.3883 79) (end 178.79 79) (width 0.2) (layer "F.Cu") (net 2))
 (segment (start 150.395 52.46) (end 151.2339 53.299) (width 0.2) (layer "F.Cu") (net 2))
 (segment (start 160.846 64.2291) (end 162.525 62.55) (width 0.2) (layer "F.Cu") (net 2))
 (segment (start 178.79 87.64) (end 177.4883 87.64) (width 0.2) (layer "F.Cu") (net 2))
 (segment (start 178.79 79) (end 180.0917 79) (width 0.2) (layer "F.Cu") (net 2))
 (segment (start 177.3883 87.54) (end 177.3883 86.52) (width 0.2) (layer "F.Cu") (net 2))
 (segment (start 144.338 68) (end 148.108 64.2291) (width 0.2) (layer "F.Cu") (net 2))
 (segment (start 162.525 59.54) (end 162.692 59.7072) (width 0.2) (layer "F.Cu") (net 2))
 (segment (start 165.911 58.9599) (end 170.551 54.32) (width 0.2) (layer "F.Cu") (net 2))
 (segment (start 165.911 59.7072) (end 165.911 58.9599) (width 0.2) (layer "F.Cu") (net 2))
 (segment (start 176 78) (end 177 79) (width 0.2) (layer "F.Cu") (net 2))
 (segment (start 170.551 54.32) (end 177.712 54.32) (width 0.2) (layer "F.Cu") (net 2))
 (segment (start 177.712 60.029) (end 177.712 65.7381) (width 0.2) (layer "B.Cu") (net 2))
 (segment (start 179.052 67.0778) (end 179.052 68.5078) (width 0.2) (layer "B.Cu") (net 2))
 (segment (start 177.7125 60.0285) (end 177.7125 54.32) (width 0.2) (layer "B.Cu") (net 2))
 (segment (start 177.712 60.029) (end 177.7125 60.0285) (width 0.2) (layer "B.Cu") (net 2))
 (segment (start 183 87.64) (end 181.7983 87.64) (width 0.2) (layer "B.Cu") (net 2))
 (segment (start 181.7983 79) (end 181.7983 87.64) (width 0.2) (layer "B.Cu") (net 2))
 (segment (start 183 79) (end 181.7983 79) (width 0.2) (layer "B.Cu") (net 2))
 (segment (start 177.712 65.7381) (end 179.052 67.0778) (width 0.2) (layer "B.Cu") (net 2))
 (segment (start 177.712 54.32) (end 177.712 60.029) (width 0.2) (layer "B.Cu") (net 2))
 (segment (start 179.052 68.5078) (end 178 69.56) (width 0.2) (layer "B.Cu") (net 2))
 (segment (start 139.354 67.7919) (end 139.646 67.5) (width 0.2) (layer "F.Cu") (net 13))
 (segment (start 139.608 69.5) (end 139.354 69.2452) (width 0.2) (layer "F.Cu") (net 13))
 (segment (start 140.425 66.5) (end 141.242 66.5) (width 0.2) (layer "F.Cu") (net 13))
 (segment (start 160.563 62.488) (end 160.625 62.55) (width 0.2) (layer "F.Cu") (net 13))
 (segment (start 141.66 62.488) (end 160.563 62.488) (width 0.2) (layer "F.Cu") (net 13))
 (segment (start 141.489 64.6513) (end 141.365 64.5273) (width 0.2) (layer "F.Cu") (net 13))
 (segment (start 139.354 69.2452) (end 139.354 67.7919) (width 0.2) (layer "F.Cu") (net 13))
 (segment (start 141.489 66.2535) (end 141.489 64.6513) (width 0.2) (layer "F.Cu") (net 13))
 (segment (start 140.425 69.5) (end 139.608 69.5) (width 0.2) (layer "F.Cu") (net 13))
 (segment (start 141.365 64.5273) (end 141.365 62.7834) (width 0.2) (layer "F.Cu") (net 13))
 (segment (start 162.175 61) (end 164.8 61) (width 0.2) (layer "F.Cu") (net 13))
 (segment (start 140.425 67) (end 140.425 66.5) (width 0.2) (layer "F.Cu") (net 13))
 (segment (start 141.365 62.7834) (end 141.66 62.488) (width 0.2) (layer "F.Cu") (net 13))
 (segment (start 139.646 67.5) (end 140.425 67.5) (width 0.2) (layer "F.Cu") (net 13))
 (segment (start 160.625 62.55) (end 162.175 61) (width 0.2) (layer "F.Cu") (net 13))
 (segment (start 140.425 67.5) (end 140.425 67) (width 0.2) (layer "F.Cu") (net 13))
 (segment (start 141.242 66.5) (end 141.489 66.2535) (width 0.2) (layer "F.Cu") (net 13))
 (segment (start 159.46 55) (end 158.308 55) (width 0.2) (layer "F.Cu") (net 6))
 (segment (start 157.038 53.73) (end 155 53.73) (width 0.2) (layer "F.Cu") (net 6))
 (segment (start 158.308 55) (end 157.038 53.73) (width 0.2) (layer "F.Cu") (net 6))
 (segment (start 159.748 53.8483) (end 159.46 53.8483) (width 0.2) (layer "B.Cu") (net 6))
 (segment (start 160.651 52.9456) (end 159.748 53.8483) (width 0.2) (layer "B.Cu") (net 6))
 (segment (start 160.651 51.9938) (end 160.651 52.9456) (width 0.2) (layer "B.Cu") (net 6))
 (segment (start 159.46 53.8483) (end 159.46 55) (width 0.2) (layer "B.Cu") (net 6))
 (segment (start 159.46 51.0717) (end 159.728 51.0717) (width 0.2) (layer "B.Cu") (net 6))
 (segment (start 159.728 51.0717) (end 160.651 51.9938) (width 0.2) (layer "B.Cu") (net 6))
 (segment (start 159.46 49.92) (end 159.46 51.0717) (width 0.2) (layer "B.Cu") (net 6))
 (segment (start 159.46 48.5317) (end 159.46 47.38) (width 0.2) (layer "F.Cu") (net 4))
 (segment (start 155 52.46) (end 158.294 52.46) (width 0.2) (layer "F.Cu") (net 4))
 (segment (start 158.294 49.4094) (end 159.172 48.5317) (width 0.2) (layer "F.Cu") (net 4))
 (segment (start 159.172 48.5317) (end 159.46 48.5317) (width 0.2) (layer "F.Cu") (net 4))
 (segment (start 158.294 52.46) (end 158.294 49.4094) (width 0.2) (layer "F.Cu") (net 4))
 (segment (start 158.294 52.46) (end 159.46 52.46) (width 0.2) (layer "F.Cu") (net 4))
 (segment (start 178.426 70.6537) (end 180.54 68.54) (width 0.2) (layer "B.Cu") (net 7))
 (segment (start 162.268 51.0717) (end 163.39 52.193) (width 0.2) (layer "B.Cu") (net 7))
 (segment (start 163.39 56.4435) (end 177.6 70.6537) (width 0.2) (layer "B.Cu") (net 7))
 (segment (start 162 49.92) (end 162 51.0717) (width 0.2) (layer "B.Cu") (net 7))
 (segment (start 163.39 52.193) (end 163.39 56.4435) (width 0.2) (layer "B.Cu") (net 7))
 (segment (start 177.6 70.6537) (end 178.426 70.6537) (width 0.2) (layer "B.Cu") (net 7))
 (segment (start 162 51.0717) (end 162.268 51.0717) (width 0.2) (layer "B.Cu") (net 7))
 (segment (start 162.268 48.5317) (end 170.135 56.3983) (width 0.2) (layer "B.Cu") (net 5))
 (segment (start 162 47.38) (end 162 48.5317) (width 0.2) (layer "B.Cu") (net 5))
 (segment (start 170.135 59.6551) (end 178 67.52) (width 0.2) (layer "B.Cu") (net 5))
 (segment (start 162 48.5317) (end 162.268 48.5317) (width 0.2) (layer "B.Cu") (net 5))
 (segment (start 170.135 56.3983) (end 170.135 59.6551) (width 0.2) (layer "B.Cu") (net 5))
 (segment (start 162 53.8483) (end 161.732 53.8483) (width 0.2) (layer "F.Cu") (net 9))
 (segment (start 160.836 52.9532) (end 160.836 51.9352) (width 0.2) (layer "F.Cu") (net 9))
 (segment (start 161.732 53.8483) (end 160.836 52.9532) (width 0.2) (layer "F.Cu") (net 9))
 (segment (start 179.657 52.705) (end 179.6575 52.705) (width 0.2) (layer "F.Cu") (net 9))
 (segment (start 162 55) (end 162 53.8483) (width 0.2) (layer "F.Cu") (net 9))
 (segment (start 161.582 51.19) (end 178.142 51.19) (width 0.2) (layer "F.Cu") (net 9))
 (segment (start 160.836 51.9352) (end 161.582 51.19) (width 0.2) (layer "F.Cu") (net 9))
 (segment (start 179.6575 52.705) (end 180.2525 53.3) (width 0.2) (layer "F.Cu") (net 9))
 (segment (start 179.657 52.705) (end 180.252 53.3) (width 0.2) (layer "F.Cu") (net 9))
 (segment (start 178.142 51.19) (end 179.657 52.705) (width 0.2) (layer "F.Cu") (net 9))
 (segment (start 162 52.46) (end 163.152 52.46) (width 0.2) (layer "F.Cu") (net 8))
 (segment (start 163.152 52.46) (end 163.332 52.28) (width 0.2) (layer "F.Cu") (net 8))
 (segment (start 163.332 52.28) (end 177.712 52.28) (width 0.2) (layer "F.Cu") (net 8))
 (segment (start 177.712 52.28) (end 177.7125 52.28) (width 0.2) (layer "F.Cu") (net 8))
 (segment (start 178.24 84.57) (end 177.3883 84.57) (width 0.2) (layer "F.Cu") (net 3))
 (segment (start 174.175 78) (end 174.175 81.3567) (width 0.2) (layer "F.Cu") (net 3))
 (segment (start 174.175 81.3567) (end 177.3883 84.57) (width 0.2) (layer "F.Cu") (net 3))
 (segment (start 177.3883 81.57) (end 176.966 81.57) (width 0.2) (layer "F.Cu") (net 1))
 (segment (start 177.5365 77.6385) (end 177.5365 78.1614) (width 0.2) (layer "F.Cu") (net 1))
 (segment (start 178.175 77) (end 177.5365 77.6385) (width 0.2) (layer "F.Cu") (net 1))
 (segment (start 178.24 81.57) (end 177.3883 81.57) (width 0.2) (layer "F.Cu") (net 1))
 (via (at 177.5365 78.1614) (size 0.6) (drill 0.3) (layers "F.Cu" "B.Cu") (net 1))
 (via (at 176.966 81.57) (size 0.6) (drill 0.3) (layers "F.Cu" "B.Cu") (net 1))
 (segment (start 176.966 78.7319) (end 177.5365 78.1614) (width 0.2) (layer "B.Cu") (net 1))
 (segment (start 176.966 81.57) (end 176.966 78.7319) (width 0.2) (layer "B.Cu") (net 1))
 (segment (start 177.6133 84.07) (end 178.24 84.07) (width 0.2) (layer "F.Cu") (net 60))
 (segment (start 177.3883 83.07) (end 177.3883 83.845) (width 0.2) (layer "F.Cu") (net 60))
 (segment (start 177.3883 83.845) (end 177.6133 84.07) (width 0.2) (layer "F.Cu") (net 60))
 (segment (start 178.24 83.07) (end 177.3883 83.07) (width 0.2) (layer "F.Cu") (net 60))
 (segment (start 179.0954 83.3628) (end 178.8882 83.57) (width 0.2) (layer "F.Cu") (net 61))
 (segment (start 178.8882 83.57) (end 178.24 83.57) (width 0.2) (layer "F.Cu") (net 61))
 (segment (start 178.24 82.57) (end 179.04 82.57) (width 0.2) (layer "F.Cu") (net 61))
 (segment (start 179.0954 82.6254) (end 179.0954 83.3628) (width 0.2) (layer "F.Cu") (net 61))
 (segment (start 179.04 82.57) (end 179.0954 82.6254) (width 0.2) (layer "F.Cu") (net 61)))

